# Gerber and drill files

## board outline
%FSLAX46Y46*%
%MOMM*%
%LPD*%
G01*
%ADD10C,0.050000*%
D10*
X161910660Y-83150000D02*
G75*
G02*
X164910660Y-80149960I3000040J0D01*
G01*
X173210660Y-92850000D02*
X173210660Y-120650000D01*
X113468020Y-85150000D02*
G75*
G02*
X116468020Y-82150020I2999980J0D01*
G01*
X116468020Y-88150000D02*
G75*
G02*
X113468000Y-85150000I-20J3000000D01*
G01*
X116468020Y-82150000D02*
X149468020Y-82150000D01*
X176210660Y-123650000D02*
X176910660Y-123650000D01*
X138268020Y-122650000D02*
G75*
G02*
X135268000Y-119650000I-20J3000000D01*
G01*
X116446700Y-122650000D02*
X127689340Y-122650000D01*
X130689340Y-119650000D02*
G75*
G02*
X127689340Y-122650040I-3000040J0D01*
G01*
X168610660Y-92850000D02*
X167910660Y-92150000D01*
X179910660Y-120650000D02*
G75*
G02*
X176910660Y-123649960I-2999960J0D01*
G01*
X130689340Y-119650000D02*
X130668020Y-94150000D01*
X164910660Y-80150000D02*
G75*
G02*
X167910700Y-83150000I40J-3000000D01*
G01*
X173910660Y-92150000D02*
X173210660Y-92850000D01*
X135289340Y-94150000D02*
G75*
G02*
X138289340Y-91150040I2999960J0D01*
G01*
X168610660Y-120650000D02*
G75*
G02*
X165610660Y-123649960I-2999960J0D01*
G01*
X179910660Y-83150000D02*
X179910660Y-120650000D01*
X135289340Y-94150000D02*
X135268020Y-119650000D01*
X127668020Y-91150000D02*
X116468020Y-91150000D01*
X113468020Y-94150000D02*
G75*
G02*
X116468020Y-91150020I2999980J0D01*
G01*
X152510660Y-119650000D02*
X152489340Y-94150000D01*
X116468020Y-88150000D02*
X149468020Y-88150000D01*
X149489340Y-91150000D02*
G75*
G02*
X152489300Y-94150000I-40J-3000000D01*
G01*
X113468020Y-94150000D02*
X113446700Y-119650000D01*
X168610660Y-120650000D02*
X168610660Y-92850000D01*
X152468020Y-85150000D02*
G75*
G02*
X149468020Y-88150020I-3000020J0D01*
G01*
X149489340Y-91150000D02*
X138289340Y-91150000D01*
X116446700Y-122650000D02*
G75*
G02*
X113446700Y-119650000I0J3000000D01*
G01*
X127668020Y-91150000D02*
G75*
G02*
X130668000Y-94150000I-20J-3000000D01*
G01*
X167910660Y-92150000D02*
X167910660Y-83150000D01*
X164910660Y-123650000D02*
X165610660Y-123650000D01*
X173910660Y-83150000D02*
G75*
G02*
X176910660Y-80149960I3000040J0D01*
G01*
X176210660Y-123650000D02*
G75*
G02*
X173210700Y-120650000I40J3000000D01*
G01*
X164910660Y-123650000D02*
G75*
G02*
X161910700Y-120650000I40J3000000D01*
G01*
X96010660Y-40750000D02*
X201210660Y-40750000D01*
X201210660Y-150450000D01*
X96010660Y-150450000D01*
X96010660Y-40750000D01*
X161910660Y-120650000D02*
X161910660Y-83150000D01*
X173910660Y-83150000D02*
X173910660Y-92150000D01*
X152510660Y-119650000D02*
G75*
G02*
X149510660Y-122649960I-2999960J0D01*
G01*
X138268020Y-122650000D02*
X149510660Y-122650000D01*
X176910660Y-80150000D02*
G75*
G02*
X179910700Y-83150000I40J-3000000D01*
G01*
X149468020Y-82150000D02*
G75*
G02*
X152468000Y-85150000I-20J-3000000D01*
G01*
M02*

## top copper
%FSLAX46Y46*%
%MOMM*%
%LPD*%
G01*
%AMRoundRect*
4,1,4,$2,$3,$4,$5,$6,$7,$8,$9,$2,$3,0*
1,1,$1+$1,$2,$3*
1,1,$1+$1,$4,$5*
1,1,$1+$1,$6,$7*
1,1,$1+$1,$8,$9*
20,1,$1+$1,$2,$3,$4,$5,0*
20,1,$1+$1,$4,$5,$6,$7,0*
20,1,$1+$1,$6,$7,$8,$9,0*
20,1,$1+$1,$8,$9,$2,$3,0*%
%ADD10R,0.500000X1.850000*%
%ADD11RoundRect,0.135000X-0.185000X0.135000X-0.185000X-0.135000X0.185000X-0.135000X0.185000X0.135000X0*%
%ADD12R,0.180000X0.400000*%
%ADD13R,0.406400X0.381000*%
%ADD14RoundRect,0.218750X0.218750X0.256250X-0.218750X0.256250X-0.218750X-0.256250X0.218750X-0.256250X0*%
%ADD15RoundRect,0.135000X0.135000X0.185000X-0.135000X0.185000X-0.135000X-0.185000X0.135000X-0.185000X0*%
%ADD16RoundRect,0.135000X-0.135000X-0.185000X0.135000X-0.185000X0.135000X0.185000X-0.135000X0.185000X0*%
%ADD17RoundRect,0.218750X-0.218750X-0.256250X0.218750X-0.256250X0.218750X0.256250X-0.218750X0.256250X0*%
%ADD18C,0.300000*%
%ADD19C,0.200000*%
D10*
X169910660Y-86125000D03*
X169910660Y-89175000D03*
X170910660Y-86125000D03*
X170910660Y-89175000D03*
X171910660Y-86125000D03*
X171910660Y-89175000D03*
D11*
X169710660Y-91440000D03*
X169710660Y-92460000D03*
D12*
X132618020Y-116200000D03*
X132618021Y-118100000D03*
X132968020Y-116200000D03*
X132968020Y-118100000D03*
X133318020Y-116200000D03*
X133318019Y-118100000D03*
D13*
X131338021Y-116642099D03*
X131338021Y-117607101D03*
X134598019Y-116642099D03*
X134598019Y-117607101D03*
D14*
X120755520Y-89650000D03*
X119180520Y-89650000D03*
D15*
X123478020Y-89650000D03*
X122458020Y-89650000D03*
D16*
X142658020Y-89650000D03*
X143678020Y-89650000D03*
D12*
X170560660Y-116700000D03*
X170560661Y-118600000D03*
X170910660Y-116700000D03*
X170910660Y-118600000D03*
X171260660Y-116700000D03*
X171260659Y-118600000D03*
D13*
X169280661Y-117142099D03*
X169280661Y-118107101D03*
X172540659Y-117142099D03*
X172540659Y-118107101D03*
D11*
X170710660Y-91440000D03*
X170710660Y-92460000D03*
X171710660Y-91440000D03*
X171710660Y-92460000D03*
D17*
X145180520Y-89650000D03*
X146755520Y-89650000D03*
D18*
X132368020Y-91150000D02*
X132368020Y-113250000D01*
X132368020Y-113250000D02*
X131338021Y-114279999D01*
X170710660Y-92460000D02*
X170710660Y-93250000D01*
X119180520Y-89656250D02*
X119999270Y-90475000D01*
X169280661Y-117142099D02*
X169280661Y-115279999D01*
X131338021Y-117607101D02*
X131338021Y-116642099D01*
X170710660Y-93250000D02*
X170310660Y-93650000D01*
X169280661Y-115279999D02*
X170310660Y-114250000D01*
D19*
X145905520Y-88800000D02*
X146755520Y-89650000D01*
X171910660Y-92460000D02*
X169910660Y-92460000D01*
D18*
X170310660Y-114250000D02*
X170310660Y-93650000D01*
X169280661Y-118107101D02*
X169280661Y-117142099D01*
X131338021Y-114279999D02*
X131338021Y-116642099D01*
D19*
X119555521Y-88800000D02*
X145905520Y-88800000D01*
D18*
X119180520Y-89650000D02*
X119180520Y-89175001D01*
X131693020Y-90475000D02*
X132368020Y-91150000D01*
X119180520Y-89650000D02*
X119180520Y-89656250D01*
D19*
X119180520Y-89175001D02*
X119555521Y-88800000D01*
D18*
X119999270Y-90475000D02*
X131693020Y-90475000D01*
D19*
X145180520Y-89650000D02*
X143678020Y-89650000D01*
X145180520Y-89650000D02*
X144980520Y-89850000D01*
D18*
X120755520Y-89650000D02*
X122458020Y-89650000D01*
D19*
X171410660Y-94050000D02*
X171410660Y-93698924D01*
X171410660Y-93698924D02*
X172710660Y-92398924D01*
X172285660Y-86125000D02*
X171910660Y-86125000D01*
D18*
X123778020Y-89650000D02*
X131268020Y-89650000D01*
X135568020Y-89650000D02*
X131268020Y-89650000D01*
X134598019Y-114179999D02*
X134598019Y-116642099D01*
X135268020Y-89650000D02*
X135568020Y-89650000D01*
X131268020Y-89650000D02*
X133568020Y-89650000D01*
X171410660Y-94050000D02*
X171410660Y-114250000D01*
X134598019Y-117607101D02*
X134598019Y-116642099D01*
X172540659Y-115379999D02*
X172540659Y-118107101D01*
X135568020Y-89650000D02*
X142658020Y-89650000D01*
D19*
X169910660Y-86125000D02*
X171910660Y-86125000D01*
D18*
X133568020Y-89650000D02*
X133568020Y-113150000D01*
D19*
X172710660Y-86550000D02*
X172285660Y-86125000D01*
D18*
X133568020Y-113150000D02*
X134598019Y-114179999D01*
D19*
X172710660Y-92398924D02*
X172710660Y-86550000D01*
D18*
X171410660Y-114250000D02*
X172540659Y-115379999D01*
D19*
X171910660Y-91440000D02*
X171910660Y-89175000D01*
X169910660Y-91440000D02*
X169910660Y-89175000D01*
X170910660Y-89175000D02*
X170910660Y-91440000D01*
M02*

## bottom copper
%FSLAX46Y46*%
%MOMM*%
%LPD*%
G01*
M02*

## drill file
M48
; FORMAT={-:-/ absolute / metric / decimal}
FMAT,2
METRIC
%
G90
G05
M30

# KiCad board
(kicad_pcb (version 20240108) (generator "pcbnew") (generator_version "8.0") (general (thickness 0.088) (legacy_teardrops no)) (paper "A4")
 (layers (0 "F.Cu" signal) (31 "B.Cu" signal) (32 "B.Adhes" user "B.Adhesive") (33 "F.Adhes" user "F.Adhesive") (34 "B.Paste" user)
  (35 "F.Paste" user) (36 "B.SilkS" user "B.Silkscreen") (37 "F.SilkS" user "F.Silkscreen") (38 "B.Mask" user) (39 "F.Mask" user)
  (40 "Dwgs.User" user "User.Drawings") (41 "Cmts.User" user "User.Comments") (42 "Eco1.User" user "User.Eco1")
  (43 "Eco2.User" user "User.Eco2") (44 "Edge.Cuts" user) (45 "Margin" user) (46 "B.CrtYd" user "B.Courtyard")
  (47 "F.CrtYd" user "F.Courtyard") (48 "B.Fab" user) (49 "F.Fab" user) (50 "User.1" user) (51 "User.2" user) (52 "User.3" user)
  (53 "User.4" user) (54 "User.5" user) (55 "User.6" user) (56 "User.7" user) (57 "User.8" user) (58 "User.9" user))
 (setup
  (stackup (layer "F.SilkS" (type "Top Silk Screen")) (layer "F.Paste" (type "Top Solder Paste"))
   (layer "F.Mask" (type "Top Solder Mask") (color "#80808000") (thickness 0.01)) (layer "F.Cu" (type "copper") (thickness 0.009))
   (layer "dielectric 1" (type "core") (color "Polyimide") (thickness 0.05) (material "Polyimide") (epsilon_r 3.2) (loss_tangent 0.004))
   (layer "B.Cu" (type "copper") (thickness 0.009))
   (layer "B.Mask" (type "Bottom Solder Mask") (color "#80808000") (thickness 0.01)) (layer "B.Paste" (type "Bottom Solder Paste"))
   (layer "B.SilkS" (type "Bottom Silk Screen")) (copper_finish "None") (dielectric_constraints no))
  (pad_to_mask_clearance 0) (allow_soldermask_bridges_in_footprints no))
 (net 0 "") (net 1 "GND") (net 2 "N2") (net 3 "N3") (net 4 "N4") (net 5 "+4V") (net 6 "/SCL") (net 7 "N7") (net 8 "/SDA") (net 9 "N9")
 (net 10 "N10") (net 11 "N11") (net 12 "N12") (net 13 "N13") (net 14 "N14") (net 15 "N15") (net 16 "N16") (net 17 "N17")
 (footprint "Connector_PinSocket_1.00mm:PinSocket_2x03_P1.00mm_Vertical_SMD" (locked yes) (layer "F.Cu") (at 170.91066 87.65 90)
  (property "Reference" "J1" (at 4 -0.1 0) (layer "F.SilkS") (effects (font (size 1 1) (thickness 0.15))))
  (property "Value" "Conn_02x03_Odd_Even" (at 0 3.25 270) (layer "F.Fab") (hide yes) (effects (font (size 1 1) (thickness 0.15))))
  (pad "1" smd rect (at 1.525 -1 90) (size 1.85 0.5) (layers "F.Cu" "F.Paste" "F.Mask") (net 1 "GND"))
  (pad "2" smd rect (at -1.525 -1 90) (size 1.85 0.5) (layers "F.Cu" "F.Paste" "F.Mask") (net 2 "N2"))
  (pad "3" smd rect (at 1.525 0 90) (size 1.85 0.5) (layers "F.Cu" "F.Paste" "F.Mask") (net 1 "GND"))
  (pad "4" smd rect (at -1.525 0 90) (size 1.85 0.5) (layers "F.Cu" "F.Paste" "F.Mask") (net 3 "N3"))
  (pad "5" smd rect (at 1.525 1 90) (size 1.85 0.5) (layers "F.Cu" "F.Paste" "F.Mask") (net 1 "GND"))
  (pad "6" smd rect (at -1.525 1 90) (size 1.85 0.5) (layers "F.Cu" "F.Paste" "F.Mask") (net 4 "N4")))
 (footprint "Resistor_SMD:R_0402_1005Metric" (layer "F.Cu") (at 169.71066 91.95 -90)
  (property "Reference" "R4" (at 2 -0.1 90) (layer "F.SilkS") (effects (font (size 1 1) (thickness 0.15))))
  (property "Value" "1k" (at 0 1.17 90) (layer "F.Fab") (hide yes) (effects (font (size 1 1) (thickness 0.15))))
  (pad "1" smd roundrect (at -0.51 0 270) (size 0.54 0.64) (layers "F.Cu" "F.Paste" "F.Mask") (roundrect_rratio 0.25) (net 2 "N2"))
  (pad "2" smd roundrect (at 0.51 0 270) (size 0.54 0.64) (layers "F.Cu" "F.Paste" "F.Mask") (roundrect_rratio 0.25) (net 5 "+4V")))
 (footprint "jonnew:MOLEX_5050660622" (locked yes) (layer "F.Cu") (at 132.96802 117.15)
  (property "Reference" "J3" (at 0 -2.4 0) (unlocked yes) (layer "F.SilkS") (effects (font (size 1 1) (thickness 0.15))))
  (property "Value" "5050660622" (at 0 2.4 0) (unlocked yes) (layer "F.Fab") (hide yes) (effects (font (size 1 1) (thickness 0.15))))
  (pad "1" smd rect (at -0.35 -0.95) (size 0.18 0.4) (layers "F.Cu" "F.Paste" "F.Mask") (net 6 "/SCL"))
  (pad "2" smd rect (at -0.349999 0.95) (size 0.18 0.4) (layers "F.Cu" "F.Paste" "F.Mask") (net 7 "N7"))
  (pad "3" smd rect (at 0 -0.95) (size 0.18 0.4) (layers "F.Cu" "F.Paste" "F.Mask") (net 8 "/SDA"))
  (pad "4" smd rect (at 0 0.95) (size 0.18 0.4) (layers "F.Cu" "F.Paste" "F.Mask") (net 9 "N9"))
  (pad "5" smd rect (at 0.35 -0.95) (size 0.18 0.4) (layers "F.Cu" "F.Paste" "F.Mask") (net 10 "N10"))
  (pad "6" smd rect (at 0.349999 0.95) (size 0.18 0.4) (layers "F.Cu" "F.Paste" "F.Mask") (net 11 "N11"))
  (pad "MP1" smd rect (at -1.629999 -0.507901) (size 0.4064 0.381) (layers "F.Cu" "F.Paste" "F.Mask") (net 5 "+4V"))
  (pad "MP2" smd rect (at -1.629999 0.457101) (size 0.4064 0.381) (layers "F.Cu" "F.Paste" "F.Mask") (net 5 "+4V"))
  (pad "MP3" smd rect (at 1.629999 -0.507901) (size 0.4064 0.381) (layers "F.Cu" "F.Paste" "F.Mask") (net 1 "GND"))
  (pad "MP4" smd rect (at 1.629999 0.457101) (size 0.4064 0.381) (layers "F.Cu" "F.Paste" "F.Mask") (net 1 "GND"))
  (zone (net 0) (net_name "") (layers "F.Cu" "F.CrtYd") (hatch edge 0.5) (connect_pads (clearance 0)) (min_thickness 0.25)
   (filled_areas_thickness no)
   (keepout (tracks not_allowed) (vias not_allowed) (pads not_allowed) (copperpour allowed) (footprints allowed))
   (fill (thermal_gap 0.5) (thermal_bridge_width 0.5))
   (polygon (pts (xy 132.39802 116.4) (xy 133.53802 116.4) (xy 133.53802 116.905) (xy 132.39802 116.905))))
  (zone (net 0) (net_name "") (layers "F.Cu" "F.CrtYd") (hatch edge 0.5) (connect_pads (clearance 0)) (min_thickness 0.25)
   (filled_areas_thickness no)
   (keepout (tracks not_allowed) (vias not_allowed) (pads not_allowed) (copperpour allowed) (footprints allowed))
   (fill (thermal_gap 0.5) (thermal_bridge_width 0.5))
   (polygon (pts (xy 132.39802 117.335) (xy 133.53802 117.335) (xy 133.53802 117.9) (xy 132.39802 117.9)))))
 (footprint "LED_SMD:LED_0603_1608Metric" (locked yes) (layer "F.Cu") (at 119.96802 89.65 180)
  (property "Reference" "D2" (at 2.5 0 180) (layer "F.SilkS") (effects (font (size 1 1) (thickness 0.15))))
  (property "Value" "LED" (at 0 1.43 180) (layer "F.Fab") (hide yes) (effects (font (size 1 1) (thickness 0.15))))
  (pad "1" smd roundrect (at -0.7875 0 180) (size 0.875 0.95) (layers "F.Cu" "F.Paste" "F.Mask") (roundrect_rratio 0.25) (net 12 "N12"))
  (pad "2" smd roundrect (at 0.7875 0 180) (size 0.875 0.95) (layers "F.Cu" "F.Paste" "F.Mask") (roundrect_rratio 0.25) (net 5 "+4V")))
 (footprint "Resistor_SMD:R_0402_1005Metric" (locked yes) (layer "F.Cu") (at 122.96802 89.65 180)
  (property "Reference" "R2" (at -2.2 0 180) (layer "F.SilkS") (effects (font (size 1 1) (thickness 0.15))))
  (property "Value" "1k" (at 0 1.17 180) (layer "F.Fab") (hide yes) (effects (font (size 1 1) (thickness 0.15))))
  (pad "1" smd roundrect (at -0.51 0 180) (size 0.54 0.64) (layers "F.Cu" "F.Paste" "F.Mask") (roundrect_rratio 0.25) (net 1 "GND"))
  (pad "2" smd roundrect (at 0.51 0 180) (size 0.54 0.64) (layers "F.Cu" "F.Paste" "F.Mask") (roundrect_rratio 0.25) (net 12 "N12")))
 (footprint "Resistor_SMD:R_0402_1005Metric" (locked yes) (layer "F.Cu") (at 143.16802 89.65)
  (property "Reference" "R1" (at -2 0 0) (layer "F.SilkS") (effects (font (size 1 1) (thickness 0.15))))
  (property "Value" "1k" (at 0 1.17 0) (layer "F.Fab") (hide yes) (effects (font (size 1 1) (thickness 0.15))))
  (pad "1" smd roundrect (at -0.51 0) (size 0.54 0.64) (layers "F.Cu" "F.Paste" "F.Mask") (roundrect_rratio 0.25) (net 1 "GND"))
  (pad "2" smd roundrect (at 0.51 0) (size 0.54 0.64) (layers "F.Cu" "F.Paste" "F.Mask") (roundrect_rratio 0.25) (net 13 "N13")))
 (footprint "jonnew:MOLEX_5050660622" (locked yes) (layer "F.Cu") (at 170.91066 117.65)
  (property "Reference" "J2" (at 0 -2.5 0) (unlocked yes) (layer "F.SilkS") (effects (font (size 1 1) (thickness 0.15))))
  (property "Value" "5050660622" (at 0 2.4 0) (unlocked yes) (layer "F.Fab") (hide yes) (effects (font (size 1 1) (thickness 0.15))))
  (pad "1" smd rect (at -0.35 -0.95) (size 0.18 0.4) (layers "F.Cu" "F.Paste" "F.Mask") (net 6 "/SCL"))
  (pad "2" smd rect (at -0.349999 0.95) (size 0.18 0.4) (layers "F.Cu" "F.Paste" "F.Mask") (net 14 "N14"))
  (pad "3" smd rect (at 0 -0.95) (size 0.18 0.4) (layers "F.Cu" "F.Paste" "F.Mask") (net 8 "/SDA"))
  (pad "4" smd rect (at 0 0.95) (size 0.18 0.4) (layers "F.Cu" "F.Paste" "F.Mask") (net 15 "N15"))
  (pad "5" smd rect (at 0.35 -0.95) (size 0.18 0.4) (layers "F.Cu" "F.Paste" "F.Mask") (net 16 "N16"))
  (pad "6" smd rect (at 0.349999 0.95) (size 0.18 0.4) (layers "F.Cu" "F.Paste" "F.Mask") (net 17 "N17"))
  (pad "MP1" smd rect (at -1.629999 -0.507901) (size 0.4064 0.381) (layers "F.Cu" "F.Paste" "F.Mask") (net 5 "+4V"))
  (pad "MP2" smd rect (at -1.629999 0.457101) (size 0.4064 0.381) (layers "F.Cu" "F.Paste" "F.Mask") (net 5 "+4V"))
  (pad "MP3" smd rect (at 1.629999 -0.507901) (size 0.4064 0.381) (layers "F.Cu" "F.Paste" "F.Mask") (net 1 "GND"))
  (pad "MP4" smd rect (at 1.629999 0.457101) (size 0.4064 0.381) (layers "F.Cu" "F.Paste" "F.Mask") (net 1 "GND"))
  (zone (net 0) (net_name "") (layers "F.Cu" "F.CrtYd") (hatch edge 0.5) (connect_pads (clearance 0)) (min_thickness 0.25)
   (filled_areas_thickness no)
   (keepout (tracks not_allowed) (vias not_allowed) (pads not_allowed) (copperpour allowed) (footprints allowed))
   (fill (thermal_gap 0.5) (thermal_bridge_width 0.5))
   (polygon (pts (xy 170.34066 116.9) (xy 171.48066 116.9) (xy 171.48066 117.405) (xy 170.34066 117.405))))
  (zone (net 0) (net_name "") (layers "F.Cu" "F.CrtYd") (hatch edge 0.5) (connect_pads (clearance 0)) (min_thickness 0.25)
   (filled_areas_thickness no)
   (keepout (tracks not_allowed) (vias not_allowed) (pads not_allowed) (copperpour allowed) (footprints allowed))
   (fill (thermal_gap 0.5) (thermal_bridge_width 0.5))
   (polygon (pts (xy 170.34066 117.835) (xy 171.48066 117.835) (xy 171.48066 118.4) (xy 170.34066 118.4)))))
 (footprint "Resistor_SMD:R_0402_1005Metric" (layer "F.Cu") (at 170.71066 91.95 -90)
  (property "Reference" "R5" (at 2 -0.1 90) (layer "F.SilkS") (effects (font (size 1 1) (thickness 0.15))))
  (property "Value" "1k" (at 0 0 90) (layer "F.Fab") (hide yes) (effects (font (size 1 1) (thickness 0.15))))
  (pad "1" smd roundrect (at -0.51 0 270) (size 0.54 0.64) (layers "F.Cu" "F.Paste" "F.Mask") (roundrect_rratio 0.25) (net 3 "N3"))
  (pad "2" smd roundrect (at 0.51 0 270) (size 0.54 0.64) (layers "F.Cu" "F.Paste" "F.Mask") (roundrect_rratio 0.25) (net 5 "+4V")))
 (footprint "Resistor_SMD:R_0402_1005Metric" (layer "F.Cu") (at 171.71066 91.95 -90)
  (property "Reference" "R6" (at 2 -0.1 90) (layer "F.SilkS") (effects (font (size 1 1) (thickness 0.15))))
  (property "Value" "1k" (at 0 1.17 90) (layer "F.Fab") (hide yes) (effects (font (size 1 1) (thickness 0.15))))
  (pad "1" smd roundrect (at -0.51 0 270) (size 0.54 0.64) (layers "F.Cu" "F.Paste" "F.Mask") (roundrect_rratio 0.25) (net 4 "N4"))
  (pad "2" smd roundrect (at 0.51 0 270) (size 0.54 0.64) (layers "F.Cu" "F.Paste" "F.Mask") (roundrect_rratio 0.25) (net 5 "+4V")))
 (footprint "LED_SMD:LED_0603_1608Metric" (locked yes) (layer "F.Cu") (at 145.96802 89.65)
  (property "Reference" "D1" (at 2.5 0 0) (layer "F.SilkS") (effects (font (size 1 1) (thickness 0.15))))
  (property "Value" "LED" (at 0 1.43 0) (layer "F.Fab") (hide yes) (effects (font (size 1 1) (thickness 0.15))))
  (pad "1" smd roundrect (at -0.7875 0) (size 0.875 0.95) (layers "F.Cu" "F.Paste" "F.Mask") (roundrect_rratio 0.25) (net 13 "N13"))
  (pad "2" smd roundrect (at 0.7875 0) (size 0.875 0.95) (layers "F.Cu" "F.Paste" "F.Mask") (roundrect_rratio 0.25) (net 5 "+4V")))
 (gr_arc (start 161.91066 83.15) (mid 162.78934 81.02868) (end 164.91066 80.15) (stroke (width 0.05) (type default)) (layer "Edge.Cuts"))
 (gr_line (start 173.21066 92.85) (end 173.21066 120.65) (stroke (width 0.05) (type default)) (layer "Edge.Cuts"))
 (gr_arc (start 113.46802 85.15) (mid 114.3467 83.02868) (end 116.46802 82.15) (stroke (width 0.05) (type default)) (layer "Edge.Cuts"))
 (gr_arc (start 116.46802 88.15) (mid 114.3467 87.27132) (end 113.46802 85.15) (stroke (width 0.05) (type default)) (layer "Edge.Cuts"))
 (gr_line (start 116.46802 82.15) (end 149.46802 82.15) (stroke (width 0.05) (type default)) (layer "Edge.Cuts"))
 (gr_line (start 176.21066 123.65) (end 176.91066 123.65) (stroke (width 0.05) (type default)) (layer "Edge.Cuts"))
 (gr_arc (start 138.26802 122.65) (mid 136.1467 121.77132) (end 135.26802 119.65) (stroke (width 0.05) (type default)) (layer "Edge.Cuts"))
 (gr_line (start 116.4467 122.65) (end 127.68934 122.65) (stroke (width 0.05) (type default)) (layer "Edge.Cuts"))
 (gr_arc (start 130.68934 119.65) (mid 129.81066 121.77132) (end 127.68934 122.65) (stroke (width 0.05) (type default)) (layer "Edge.Cuts"))
 (gr_line (start 168.61066 92.85) (end 167.91066 92.15) (stroke (width 0.05) (type default)) (layer "Edge.Cuts"))
 (gr_arc (start 179.91066 120.65) (mid 179.03198 122.77132) (end 176.91066 123.65) (stroke (width 0.05) (type default)) (layer "Edge.Cuts"))
 (gr_line (start 130.68934 119.65) (end 130.66802 94.15) (stroke (width 0.05) (type default)) (layer "Edge.Cuts"))
 (gr_arc (start 164.91066 80.15) (mid 167.03198 81.02868) (end 167.91066 83.15) (stroke (width 0.05) (type default)) (layer "Edge.Cuts"))
 (gr_line (start 173.91066 92.15) (end 173.21066 92.85) (stroke (width 0.05) (type default)) (layer "Edge.Cuts"))
 (gr_arc (start 135.28934 94.15) (mid 136.16802 92.02868) (end 138.28934 91.15) (stroke (width 0.05) (type default)) (layer "Edge.Cuts"))
 (gr_arc (start 168.61066 120.65) (mid 167.73198 122.77132) (end 165.61066 123.65) (stroke (width 0.05) (type default)) (layer "Edge.Cuts"))
 (gr_line (start 179.91066 83.15) (end 179.91066 120.65) (stroke (width 0.05) (type default)) (layer "Edge.Cuts"))
 (gr_line (start 135.28934 94.15) (end 135.26802 119.65) (stroke (width 0.05) (type default)) (layer "Edge.Cuts"))
 (gr_line (start 127.66802 91.15) (end 116.46802 91.15) (stroke (width 0.05) (type default)) (layer "Edge.Cuts"))
 (gr_arc (start 113.46802 94.15) (mid 114.3467 92.02868) (end 116.46802 91.15) (stroke (width 0.05) (type default)) (layer "Edge.Cuts"))
 (gr_line (start 152.51066 119.65) (end 152.48934 94.15) (stroke (width 0.05) (type default)) (layer "Edge.Cuts"))
 (gr_line (start 116.46802 88.15) (end 149.46802 88.15) (stroke (width 0.05) (type default)) (layer "Edge.Cuts"))
 (gr_arc (start 149.48934 91.15) (mid 151.61066 92.02868) (end 152.48934 94.15) (stroke (width 0.05) (type default)) (layer "Edge.Cuts"))
 (gr_line (start 113.46802 94.15) (end 113.4467 119.65) (stroke (width 0.05) (type default)) (layer "Edge.Cuts"))
 (gr_line (start 168.61066 120.65) (end 168.61066 92.85) (stroke (width 0.05) (type default)) (layer "Edge.Cuts"))
 (gr_arc (start 152.46802 85.15) (mid 151.58934 87.27132) (end 149.46802 88.15) (stroke (width 0.05) (type default)) (layer "Edge.Cuts"))
 (gr_line (start 149.48934 91.15) (end 138.28934 91.15) (stroke (width 0.05) (type default)) (layer "Edge.Cuts"))
 (gr_arc (start 116.4467 122.65) (mid 114.32538 121.77132) (end 113.4467 119.65) (stroke (width 0.05) (type default)) (layer "Edge.Cuts"))
 (gr_arc (start 127.66802 91.15) (mid 129.78934 92.02868) (end 130.66802 94.15) (stroke (width 0.05) (type default)) (layer "Edge.Cuts"))
 (gr_line (start 167.91066 92.15) (end 167.91066 83.15) (stroke (width 0.05) (type default)) (layer "Edge.Cuts"))
 (gr_line (start 164.91066 123.65) (end 165.61066 123.65) (stroke (width 0.05) (type default)) (layer "Edge.Cuts"))
 (gr_arc (start 173.91066 83.15) (mid 174.78934 81.02868) (end 176.91066 80.15) (stroke (width 0.05) (type default)) (layer "Edge.Cuts"))
 (gr_arc (start 176.21066 123.65) (mid 174.08934 122.77132) (end 173.21066 120.65) (stroke (width 0.05) (type default)) (layer "Edge.Cuts"))
 (gr_arc (start 164.91066 123.65) (mid 162.78934 122.77132) (end 161.91066 120.65) (stroke (width 0.05) (type default)) (layer "Edge.Cuts"))
 (gr_rect (start 96.01066 40.75) (end 201.21066 150.45) (stroke (width 0.05) (type default)) (fill none) (layer "Edge.Cuts"))
 (gr_line (start 161.91066 120.65) (end 161.91066 83.15) (stroke (width 0.05) (type default)) (layer "Edge.Cuts"))
 (gr_line (start 173.91066 83.15) (end 173.91066 92.15) (stroke (width 0.05) (type default)) (layer "Edge.Cuts"))
 (gr_arc (start 152.51066 119.65) (mid 151.63198 121.77132) (end 149.51066 122.65) (stroke (width 0.05) (type default)) (layer "Edge.Cuts"))
 (gr_line (start 138.26802 122.65) (end 149.51066 122.65) (stroke (width 0.05) (type default)) (layer "Edge.Cuts"))
 (gr_arc (start 176.91066 80.15) (mid 179.03198 81.02868) (end 179.91066 83.15) (stroke (width 0.05) (type default)) (layer "Edge.Cuts"))
 (gr_arc (start 149.46802 82.15) (mid 151.58934 83.02868) (end 152.46802 85.15) (stroke (width 0.05) (type default)) (layer "Edge.Cuts"))
 (segment (start 132.36802 91.15) (end 132.36802 113.25) (width 0.3) (layer "F.Cu") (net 5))
 (segment (start 132.36802 113.25) (end 131.338021 114.279999) (width 0.3) (layer "F.Cu") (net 5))
 (segment (start 170.71066 92.46) (end 170.71066 93.25) (width 0.3) (layer "F.Cu") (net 5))
 (segment (start 119.18052 89.65625) (end 119.99927 90.475) (width 0.3) (layer "F.Cu") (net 5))
 (segment (start 169.280661 117.142099) (end 169.280661 115.279999) (width 0.3) (layer "F.Cu") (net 5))
 (segment (start 131.338021 117.607101) (end 131.338021 116.642099) (width 0.3) (layer "F.Cu") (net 5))
 (segment (start 170.71066 93.25) (end 170.31066 93.65) (width 0.3) (layer "F.Cu") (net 5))
 (segment (start 169.280661 115.279999) (end 170.31066 114.25) (width 0.3) (layer "F.Cu") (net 5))
 (segment (start 145.90552 88.8) (end 146.75552 89.65) (width 0.2) (layer "F.Cu") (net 5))
 (segment (start 171.91066 92.46) (end 169.91066 92.46) (width 0.2) (layer "F.Cu") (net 5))
 (segment (start 170.31066 114.25) (end 170.31066 93.65) (width 0.3) (layer "F.Cu") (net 5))
 (segment (start 169.280661 118.107101) (end 169.280661 117.142099) (width 0.3) (layer "F.Cu") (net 5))
 (segment (start 131.338021 114.279999) (end 131.338021 116.642099) (width 0.3) (layer "F.Cu") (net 5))
 (segment (start 119.555521 88.8) (end 145.90552 88.8) (width 0.2) (layer "F.Cu") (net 5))
 (segment (start 119.18052 89.65) (end 119.18052 89.175001) (width 0.3) (layer "F.Cu") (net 5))
 (segment (start 131.69302 90.475) (end 132.36802 91.15) (width 0.3) (layer "F.Cu") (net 5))
 (segment (start 119.18052 89.65) (end 119.18052 89.65625) (width 0.3) (layer "F.Cu") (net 5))
 (segment (start 119.18052 89.175001) (end 119.555521 88.8) (width 0.2) (layer "F.Cu") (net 5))
 (segment (start 119.99927 90.475) (end 131.69302 90.475) (width 0.3) (layer "F.Cu") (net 5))
 (segment (start 145.18052 89.65) (end 143.67802 89.65) (width 0.2) (layer "F.Cu") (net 13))
 (segment (start 145.18052 89.65) (end 144.98052 89.85) (width 0.2) (layer "F.Cu") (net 13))
 (segment (start 120.75552 89.65) (end 122.45802 89.65) (width 0.3) (layer "F.Cu") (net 12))
 (segment (start 171.41066 94.05) (end 171.41066 93.698924) (width 0.2) (layer "F.Cu") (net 1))
 (segment (start 171.41066 93.698924) (end 172.71066 92.398924) (width 0.2) (layer "F.Cu") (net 1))
 (segment (start 172.28566 86.125) (end 171.91066 86.125) (width 0.2) (layer "F.Cu") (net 1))
 (segment (start 123.77802 89.65) (end 131.26802 89.65) (width 0.3) (layer "F.Cu") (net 1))
 (segment (start 135.56802 89.65) (end 131.26802 89.65) (width 0.3) (layer "F.Cu") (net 1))
 (segment (start 134.598019 114.179999) (end 134.598019 116.642099) (width 0.3) (layer "F.Cu") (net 1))
 (segment (start 135.26802 89.65) (end 135.56802 89.65) (width 0.3) (layer "F.Cu") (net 1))
 (segment (start 131.26802 89.65) (end 133.56802 89.65) (width 0.3) (layer "F.Cu") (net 1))
 (segment (start 171.41066 94.05) (end 171.41066 114.25) (width 0.3) (layer "F.Cu") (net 1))
 (segment (start 134.598019 117.607101) (end 134.598019 116.642099) (width 0.3) (layer "F.Cu") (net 1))
 (segment (start 172.540659 115.379999) (end 172.540659 118.107101) (width 0.3) (layer "F.Cu") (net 1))
 (segment (start 135.56802 89.65) (end 142.65802 89.65) (width 0.3) (layer "F.Cu") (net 1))
 (segment (start 169.91066 86.125) (end 171.91066 86.125) (width 0.2) (layer "F.Cu") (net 1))
 (segment (start 133.56802 89.65) (end 133.56802 113.15) (width 0.3) (layer "F.Cu") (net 1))
 (segment (start 172.71066 86.55) (end 172.28566 86.125) (width 0.2) (layer "F.Cu") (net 1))
 (segment (start 133.56802 113.15) (end 134.598019 114.179999) (width 0.3) (layer "F.Cu") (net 1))
 (segment (start 172.71066 92.398924) (end 172.71066 86.55) (width 0.2) (layer "F.Cu") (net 1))
 (segment (start 171.41066 114.25) (end 172.540659 115.379999) (width 0.3) (layer "F.Cu") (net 1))
 (segment (start 171.91066 91.44) (end 171.91066 89.175) (width 0.2) (layer "F.Cu") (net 4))
 (segment (start 169.91066 91.44) (end 169.91066 89.175) (width 0.2) (layer "F.Cu") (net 2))
 (segment (start 170.91066 89.175) (end 170.91066 91.44) (width 0.2) (layer "F.Cu") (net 3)))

